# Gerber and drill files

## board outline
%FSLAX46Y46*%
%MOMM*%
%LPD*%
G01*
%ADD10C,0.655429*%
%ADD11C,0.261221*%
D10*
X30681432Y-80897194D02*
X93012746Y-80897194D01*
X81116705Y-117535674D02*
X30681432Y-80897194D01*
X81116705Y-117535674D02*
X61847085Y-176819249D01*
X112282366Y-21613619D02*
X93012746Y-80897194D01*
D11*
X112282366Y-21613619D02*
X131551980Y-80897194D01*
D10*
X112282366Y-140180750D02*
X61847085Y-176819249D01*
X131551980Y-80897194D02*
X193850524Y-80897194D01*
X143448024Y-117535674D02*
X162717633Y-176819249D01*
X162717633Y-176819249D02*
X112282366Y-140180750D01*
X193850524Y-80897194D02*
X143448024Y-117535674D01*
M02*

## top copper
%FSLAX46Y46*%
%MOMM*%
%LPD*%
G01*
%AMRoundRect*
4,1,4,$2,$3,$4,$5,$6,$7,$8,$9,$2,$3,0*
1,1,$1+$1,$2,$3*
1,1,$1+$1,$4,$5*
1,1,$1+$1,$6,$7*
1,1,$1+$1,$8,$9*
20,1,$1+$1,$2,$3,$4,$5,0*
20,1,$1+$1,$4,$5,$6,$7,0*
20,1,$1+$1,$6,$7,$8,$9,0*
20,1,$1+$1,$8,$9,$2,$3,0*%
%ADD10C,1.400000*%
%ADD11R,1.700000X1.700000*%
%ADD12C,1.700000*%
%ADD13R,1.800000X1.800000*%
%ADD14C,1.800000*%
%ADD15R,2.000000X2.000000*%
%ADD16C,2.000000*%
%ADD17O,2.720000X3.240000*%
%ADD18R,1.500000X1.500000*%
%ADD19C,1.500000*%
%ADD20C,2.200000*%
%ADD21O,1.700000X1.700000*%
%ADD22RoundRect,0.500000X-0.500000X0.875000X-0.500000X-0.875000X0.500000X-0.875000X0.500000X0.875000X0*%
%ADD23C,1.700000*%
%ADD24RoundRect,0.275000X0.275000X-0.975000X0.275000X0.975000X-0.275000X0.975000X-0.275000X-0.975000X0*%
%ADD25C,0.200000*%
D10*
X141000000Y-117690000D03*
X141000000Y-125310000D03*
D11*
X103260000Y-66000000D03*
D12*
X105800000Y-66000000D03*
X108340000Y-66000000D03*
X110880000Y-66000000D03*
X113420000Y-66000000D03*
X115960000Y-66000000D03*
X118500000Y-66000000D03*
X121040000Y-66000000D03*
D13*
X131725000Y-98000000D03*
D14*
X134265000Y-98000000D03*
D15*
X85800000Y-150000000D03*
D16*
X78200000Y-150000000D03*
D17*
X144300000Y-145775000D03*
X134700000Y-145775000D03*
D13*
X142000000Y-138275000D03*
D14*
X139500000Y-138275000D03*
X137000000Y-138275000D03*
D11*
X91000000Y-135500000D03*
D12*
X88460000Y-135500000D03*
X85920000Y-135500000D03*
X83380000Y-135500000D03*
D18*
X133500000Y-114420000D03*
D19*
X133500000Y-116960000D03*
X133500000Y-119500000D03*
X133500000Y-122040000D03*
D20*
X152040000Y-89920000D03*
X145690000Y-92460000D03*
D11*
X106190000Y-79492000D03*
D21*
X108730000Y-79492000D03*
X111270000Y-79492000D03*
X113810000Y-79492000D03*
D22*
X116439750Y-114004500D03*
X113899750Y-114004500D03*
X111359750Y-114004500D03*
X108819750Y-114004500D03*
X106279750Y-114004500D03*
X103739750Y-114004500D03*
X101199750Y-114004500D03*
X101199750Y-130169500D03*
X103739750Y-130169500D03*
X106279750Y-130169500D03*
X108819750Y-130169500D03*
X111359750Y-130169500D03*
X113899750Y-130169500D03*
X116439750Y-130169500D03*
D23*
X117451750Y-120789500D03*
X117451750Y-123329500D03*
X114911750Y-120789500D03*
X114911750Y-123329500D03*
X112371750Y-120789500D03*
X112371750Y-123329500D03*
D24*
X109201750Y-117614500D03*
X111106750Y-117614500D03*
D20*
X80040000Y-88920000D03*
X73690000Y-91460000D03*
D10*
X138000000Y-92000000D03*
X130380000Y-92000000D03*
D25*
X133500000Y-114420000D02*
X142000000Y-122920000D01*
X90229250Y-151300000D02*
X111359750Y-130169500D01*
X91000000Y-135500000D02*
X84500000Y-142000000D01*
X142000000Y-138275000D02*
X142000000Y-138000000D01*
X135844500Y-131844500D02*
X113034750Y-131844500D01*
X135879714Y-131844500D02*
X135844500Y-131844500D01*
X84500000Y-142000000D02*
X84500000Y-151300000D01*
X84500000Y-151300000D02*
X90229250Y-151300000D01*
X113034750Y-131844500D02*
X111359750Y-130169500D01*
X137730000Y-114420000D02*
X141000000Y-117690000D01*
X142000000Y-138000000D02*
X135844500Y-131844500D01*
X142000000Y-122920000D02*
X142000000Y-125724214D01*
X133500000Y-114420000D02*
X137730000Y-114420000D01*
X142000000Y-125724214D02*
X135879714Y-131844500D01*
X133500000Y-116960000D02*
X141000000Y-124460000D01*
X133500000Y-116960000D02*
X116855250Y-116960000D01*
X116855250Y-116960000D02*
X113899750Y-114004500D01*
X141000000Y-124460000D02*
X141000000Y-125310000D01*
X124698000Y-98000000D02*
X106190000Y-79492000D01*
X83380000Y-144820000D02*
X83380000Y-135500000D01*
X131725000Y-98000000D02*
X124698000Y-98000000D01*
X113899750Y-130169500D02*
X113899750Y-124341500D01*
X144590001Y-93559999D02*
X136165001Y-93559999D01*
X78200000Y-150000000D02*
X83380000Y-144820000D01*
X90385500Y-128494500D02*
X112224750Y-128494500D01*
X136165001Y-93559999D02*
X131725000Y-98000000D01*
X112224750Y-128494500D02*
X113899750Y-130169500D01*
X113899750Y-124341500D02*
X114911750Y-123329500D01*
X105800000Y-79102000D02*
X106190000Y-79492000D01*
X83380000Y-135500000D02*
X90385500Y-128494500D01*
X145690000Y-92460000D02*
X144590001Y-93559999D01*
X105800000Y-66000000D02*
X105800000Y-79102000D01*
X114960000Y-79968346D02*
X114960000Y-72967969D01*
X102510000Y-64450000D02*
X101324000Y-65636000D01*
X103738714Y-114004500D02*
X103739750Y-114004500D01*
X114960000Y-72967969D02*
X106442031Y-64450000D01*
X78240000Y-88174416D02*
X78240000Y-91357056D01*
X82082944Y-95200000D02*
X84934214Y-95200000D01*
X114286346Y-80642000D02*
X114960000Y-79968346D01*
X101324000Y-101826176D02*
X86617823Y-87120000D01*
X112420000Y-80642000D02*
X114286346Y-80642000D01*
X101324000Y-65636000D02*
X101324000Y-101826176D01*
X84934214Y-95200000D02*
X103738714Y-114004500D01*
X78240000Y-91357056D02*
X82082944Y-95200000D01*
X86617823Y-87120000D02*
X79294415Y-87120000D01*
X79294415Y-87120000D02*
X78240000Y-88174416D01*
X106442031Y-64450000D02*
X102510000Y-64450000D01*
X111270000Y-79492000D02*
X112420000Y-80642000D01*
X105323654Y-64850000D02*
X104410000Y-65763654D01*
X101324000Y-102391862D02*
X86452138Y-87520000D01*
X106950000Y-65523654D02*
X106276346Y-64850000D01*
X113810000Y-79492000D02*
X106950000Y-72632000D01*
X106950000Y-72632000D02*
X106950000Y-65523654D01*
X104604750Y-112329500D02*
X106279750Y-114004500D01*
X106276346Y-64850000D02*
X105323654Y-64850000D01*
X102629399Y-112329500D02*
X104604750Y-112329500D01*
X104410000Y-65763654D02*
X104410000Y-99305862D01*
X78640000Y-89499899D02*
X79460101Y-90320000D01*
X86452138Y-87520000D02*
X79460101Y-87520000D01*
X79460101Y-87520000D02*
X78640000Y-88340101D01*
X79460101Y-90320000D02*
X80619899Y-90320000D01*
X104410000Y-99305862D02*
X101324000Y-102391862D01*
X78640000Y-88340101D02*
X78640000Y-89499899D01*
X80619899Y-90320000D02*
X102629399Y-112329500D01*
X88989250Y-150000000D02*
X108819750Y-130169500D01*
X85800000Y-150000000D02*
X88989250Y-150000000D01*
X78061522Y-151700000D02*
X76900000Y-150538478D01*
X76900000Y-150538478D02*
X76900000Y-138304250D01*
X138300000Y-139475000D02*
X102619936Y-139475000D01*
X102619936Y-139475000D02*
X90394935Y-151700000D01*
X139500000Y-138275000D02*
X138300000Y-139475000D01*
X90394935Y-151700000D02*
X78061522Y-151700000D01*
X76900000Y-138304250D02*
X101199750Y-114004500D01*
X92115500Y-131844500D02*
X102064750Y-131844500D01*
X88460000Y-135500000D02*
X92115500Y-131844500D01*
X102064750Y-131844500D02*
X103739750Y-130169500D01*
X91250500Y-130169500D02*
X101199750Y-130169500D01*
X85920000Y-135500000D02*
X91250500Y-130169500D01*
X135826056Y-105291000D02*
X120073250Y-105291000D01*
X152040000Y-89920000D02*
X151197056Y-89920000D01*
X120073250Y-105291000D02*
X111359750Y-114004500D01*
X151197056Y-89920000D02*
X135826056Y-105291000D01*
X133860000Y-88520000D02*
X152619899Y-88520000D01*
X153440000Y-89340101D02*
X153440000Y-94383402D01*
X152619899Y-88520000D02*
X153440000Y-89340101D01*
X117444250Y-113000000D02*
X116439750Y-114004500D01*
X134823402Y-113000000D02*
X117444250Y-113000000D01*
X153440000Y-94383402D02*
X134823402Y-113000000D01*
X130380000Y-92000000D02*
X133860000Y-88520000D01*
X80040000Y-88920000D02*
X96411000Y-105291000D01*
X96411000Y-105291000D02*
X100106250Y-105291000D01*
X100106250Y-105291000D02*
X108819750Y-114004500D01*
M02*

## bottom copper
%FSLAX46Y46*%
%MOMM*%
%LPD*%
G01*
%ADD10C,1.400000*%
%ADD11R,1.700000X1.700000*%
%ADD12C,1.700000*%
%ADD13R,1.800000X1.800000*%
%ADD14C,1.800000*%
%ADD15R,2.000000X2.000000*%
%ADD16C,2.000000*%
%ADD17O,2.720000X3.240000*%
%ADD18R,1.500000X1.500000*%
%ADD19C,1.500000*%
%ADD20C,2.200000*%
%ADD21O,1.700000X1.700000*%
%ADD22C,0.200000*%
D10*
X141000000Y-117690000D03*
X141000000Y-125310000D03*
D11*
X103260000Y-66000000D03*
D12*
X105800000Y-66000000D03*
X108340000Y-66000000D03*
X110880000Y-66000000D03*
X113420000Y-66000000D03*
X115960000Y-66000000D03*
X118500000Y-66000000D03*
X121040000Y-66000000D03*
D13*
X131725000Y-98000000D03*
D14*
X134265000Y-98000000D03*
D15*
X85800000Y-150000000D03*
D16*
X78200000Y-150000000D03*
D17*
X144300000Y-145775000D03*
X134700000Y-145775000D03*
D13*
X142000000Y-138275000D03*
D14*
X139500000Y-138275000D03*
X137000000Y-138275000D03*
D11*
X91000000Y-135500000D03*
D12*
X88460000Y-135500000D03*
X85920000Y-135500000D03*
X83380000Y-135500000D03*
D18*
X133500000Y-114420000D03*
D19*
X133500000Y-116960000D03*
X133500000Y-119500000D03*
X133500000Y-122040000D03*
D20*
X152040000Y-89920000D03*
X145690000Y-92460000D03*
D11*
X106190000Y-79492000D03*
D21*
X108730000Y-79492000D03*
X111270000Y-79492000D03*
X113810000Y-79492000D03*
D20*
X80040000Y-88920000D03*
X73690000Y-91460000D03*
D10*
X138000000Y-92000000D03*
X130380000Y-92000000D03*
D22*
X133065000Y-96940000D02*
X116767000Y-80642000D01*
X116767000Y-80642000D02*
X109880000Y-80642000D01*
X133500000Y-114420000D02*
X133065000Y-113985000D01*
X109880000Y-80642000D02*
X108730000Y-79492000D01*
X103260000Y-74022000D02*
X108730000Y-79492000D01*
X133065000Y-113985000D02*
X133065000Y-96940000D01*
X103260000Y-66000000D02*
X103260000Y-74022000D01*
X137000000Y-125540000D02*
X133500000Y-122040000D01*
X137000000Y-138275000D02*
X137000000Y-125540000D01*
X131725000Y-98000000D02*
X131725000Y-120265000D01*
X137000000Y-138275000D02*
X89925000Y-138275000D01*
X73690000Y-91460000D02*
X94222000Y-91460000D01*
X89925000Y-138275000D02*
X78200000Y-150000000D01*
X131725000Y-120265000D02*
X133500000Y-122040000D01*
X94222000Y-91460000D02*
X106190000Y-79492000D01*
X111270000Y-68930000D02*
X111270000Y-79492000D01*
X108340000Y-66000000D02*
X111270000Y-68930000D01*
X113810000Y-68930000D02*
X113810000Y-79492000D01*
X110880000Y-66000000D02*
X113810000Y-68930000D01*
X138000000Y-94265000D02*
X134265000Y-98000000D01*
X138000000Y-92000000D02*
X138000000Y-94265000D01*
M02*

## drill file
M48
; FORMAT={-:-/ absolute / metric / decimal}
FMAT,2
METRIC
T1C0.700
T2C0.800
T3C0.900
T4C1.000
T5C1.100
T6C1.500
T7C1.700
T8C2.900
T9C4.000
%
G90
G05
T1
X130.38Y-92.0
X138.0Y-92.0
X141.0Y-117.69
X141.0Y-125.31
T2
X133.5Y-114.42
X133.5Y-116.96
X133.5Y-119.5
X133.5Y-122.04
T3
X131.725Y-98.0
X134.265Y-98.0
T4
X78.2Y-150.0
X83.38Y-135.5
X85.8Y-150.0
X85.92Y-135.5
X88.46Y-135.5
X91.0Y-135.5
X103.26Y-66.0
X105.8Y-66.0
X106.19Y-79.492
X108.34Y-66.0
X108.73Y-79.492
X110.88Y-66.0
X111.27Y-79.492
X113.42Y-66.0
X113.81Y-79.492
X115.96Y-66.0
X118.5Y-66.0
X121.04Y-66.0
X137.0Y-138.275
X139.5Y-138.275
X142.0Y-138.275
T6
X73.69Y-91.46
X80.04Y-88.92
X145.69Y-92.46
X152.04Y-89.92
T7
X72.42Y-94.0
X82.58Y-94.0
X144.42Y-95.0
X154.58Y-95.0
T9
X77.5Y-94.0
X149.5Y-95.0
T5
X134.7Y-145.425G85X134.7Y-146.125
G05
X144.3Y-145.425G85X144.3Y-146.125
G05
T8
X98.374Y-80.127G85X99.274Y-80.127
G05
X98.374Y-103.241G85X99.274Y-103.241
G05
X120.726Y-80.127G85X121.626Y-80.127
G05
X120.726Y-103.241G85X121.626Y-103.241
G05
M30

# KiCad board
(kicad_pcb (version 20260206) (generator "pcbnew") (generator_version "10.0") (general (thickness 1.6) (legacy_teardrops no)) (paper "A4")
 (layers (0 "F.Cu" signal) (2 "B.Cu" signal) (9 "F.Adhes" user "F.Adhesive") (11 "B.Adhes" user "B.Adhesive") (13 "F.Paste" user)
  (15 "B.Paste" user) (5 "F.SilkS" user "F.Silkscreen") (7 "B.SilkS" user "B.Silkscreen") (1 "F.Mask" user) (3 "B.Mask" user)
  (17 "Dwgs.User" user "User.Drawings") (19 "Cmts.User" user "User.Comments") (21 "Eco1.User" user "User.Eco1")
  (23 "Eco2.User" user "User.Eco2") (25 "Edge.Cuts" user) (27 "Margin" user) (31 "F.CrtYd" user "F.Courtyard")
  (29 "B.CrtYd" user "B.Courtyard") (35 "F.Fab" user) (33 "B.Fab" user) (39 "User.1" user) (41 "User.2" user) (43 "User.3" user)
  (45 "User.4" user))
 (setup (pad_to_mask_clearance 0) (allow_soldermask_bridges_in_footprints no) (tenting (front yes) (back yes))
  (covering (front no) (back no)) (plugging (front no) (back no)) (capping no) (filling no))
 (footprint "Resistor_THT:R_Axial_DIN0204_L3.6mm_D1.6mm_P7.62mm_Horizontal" (layer "F.Cu") (at 141 117.69 -90)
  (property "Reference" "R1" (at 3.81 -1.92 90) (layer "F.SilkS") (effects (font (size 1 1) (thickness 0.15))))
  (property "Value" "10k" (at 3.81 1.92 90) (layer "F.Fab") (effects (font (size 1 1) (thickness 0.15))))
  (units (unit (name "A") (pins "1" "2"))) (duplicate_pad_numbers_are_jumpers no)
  (pad "1" thru_hole circle (at 0 0 270) (size 1.4 1.4) (drill 0.7) (layers "*.Cu" "*.Mask") (remove_unused_layers no) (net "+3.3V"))
  (pad "2" thru_hole circle (at 7.62 0 270) (size 1.4 1.4) (drill 0.7) (layers "*.Cu" "*.Mask") (remove_unused_layers no)
   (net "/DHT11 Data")))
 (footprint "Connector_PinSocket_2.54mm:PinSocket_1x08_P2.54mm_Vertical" (layer "F.Cu") (at 103.26 66 90)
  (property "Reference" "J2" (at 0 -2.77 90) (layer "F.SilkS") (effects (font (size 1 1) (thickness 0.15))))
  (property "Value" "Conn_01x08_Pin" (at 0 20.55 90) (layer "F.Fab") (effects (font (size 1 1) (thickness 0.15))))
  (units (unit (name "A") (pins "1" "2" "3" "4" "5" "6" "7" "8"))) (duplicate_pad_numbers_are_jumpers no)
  (pad "1" thru_hole rect (at 0 0 90) (size 1.7 1.7) (drill 1) (layers "*.Cu" "*.Mask") (remove_unused_layers no) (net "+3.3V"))
  (pad "2" thru_hole circle (at 0 2.54 90) (size 1.7 1.7) (drill 1) (layers "*.Cu" "*.Mask") (remove_unused_layers no) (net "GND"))
  (pad "3" thru_hole circle (at 0 5.08 90) (size 1.7 1.7) (drill 1) (layers "*.Cu" "*.Mask") (remove_unused_layers no) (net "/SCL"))
  (pad "4" thru_hole circle (at 0 7.62 90) (size 1.7 1.7) (drill 1) (layers "*.Cu" "*.Mask") (remove_unused_layers no) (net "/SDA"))
  (pad "5" thru_hole circle (at 0 10.16 90) (size 1.7 1.7) (drill 1) (layers "*.Cu" "*.Mask") (remove_unused_layers no)
   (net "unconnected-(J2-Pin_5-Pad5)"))
  (pad "6" thru_hole circle (at 0 12.7 90) (size 1.7 1.7) (drill 1) (layers "*.Cu" "*.Mask") (remove_unused_layers no)
   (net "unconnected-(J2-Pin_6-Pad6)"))
  (pad "7" thru_hole circle (at 0 15.24 90) (size 1.7 1.7) (drill 1) (layers "*.Cu" "*.Mask") (remove_unused_layers no)
   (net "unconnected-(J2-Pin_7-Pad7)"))
  (pad "8" thru_hole circle (at 0 17.78 90) (size 1.7 1.7) (drill 1) (layers "*.Cu" "*.Mask") (remove_unused_layers no)
   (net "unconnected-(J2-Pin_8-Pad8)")))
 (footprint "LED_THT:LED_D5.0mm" (layer "F.Cu") (at 131.725 98)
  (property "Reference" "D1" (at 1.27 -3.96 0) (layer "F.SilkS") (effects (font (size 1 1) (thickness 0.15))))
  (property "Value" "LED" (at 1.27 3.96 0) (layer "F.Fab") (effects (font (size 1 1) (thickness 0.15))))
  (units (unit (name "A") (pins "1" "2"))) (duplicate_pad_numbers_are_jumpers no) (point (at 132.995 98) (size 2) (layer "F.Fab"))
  (pad "1" thru_hole rect (at 0 0) (size 1.8 1.8) (drill 0.9) (layers "*.Cu" "*.Mask") (remove_unused_layers no) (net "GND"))
  (pad "2" thru_hole circle (at 2.54 0) (size 1.8 1.8) (drill 0.9) (layers "*.Cu" "*.Mask") (remove_unused_layers no) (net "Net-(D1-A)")))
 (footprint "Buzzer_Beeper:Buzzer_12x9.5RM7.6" (layer "F.Cu") (at 85.8 150 180)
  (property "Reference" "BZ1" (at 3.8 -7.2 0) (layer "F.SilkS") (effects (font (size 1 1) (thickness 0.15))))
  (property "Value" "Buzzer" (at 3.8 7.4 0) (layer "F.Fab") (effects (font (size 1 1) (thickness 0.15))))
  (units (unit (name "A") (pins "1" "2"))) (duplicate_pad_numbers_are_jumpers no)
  (pad "1" thru_hole rect (at 0 0 180) (size 2 2) (drill 1) (layers "*.Cu" "*.Mask") (remove_unused_layers no) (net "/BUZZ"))
  (pad "2" thru_hole circle (at 7.6 0 180) (size 2 2) (drill 1) (layers "*.Cu" "*.Mask") (remove_unused_layers no) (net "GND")))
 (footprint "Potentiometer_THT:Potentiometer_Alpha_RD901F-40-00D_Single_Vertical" (layer "F.Cu") (at 142 138.275 -90)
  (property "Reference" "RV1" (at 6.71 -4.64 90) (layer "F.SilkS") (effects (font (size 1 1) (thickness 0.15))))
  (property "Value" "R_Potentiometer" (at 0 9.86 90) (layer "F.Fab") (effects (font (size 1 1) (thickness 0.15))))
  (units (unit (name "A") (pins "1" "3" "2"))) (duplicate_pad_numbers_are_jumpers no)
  (pad "" thru_hole oval (at 7.5 -2.3) (size 2.72 3.24) (drill oval 1.1 1.8) (layers "*.Cu" "*.Mask") (remove_unused_layers no))
  (pad "" thru_hole oval (at 7.5 7.3) (size 2.72 3.24) (drill oval 1.1 1.8) (layers "*.Cu" "*.Mask") (remove_unused_layers no))
  (pad "1" thru_hole rect (at 0 0) (size 1.8 1.8) (drill 1) (layers "*.Cu" "*.Mask") (remove_unused_layers no) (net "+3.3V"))
  (pad "2" thru_hole circle (at 0 2.5) (size 1.8 1.8) (drill 1) (layers "*.Cu" "*.Mask") (remove_unused_layers no) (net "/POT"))
  (pad "3" thru_hole circle (at 0 5) (size 1.8 1.8) (drill 1) (layers "*.Cu" "*.Mask") (remove_unused_layers no) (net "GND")))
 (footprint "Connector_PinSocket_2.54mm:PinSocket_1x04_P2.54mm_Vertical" (layer "F.Cu") (at 91 135.5 -90)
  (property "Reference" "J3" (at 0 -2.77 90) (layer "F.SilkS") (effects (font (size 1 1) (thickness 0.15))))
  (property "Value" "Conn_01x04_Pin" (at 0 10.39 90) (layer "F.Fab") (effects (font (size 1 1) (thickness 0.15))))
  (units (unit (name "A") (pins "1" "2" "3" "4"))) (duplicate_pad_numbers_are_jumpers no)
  (pad "1" thru_hole rect (at 0 0 270) (size 1.7 1.7) (drill 1) (layers "*.Cu" "*.Mask") (remove_unused_layers no) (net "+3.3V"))
  (pad "2" thru_hole circle (at 0 2.54 270) (size 1.7 1.7) (drill 1) (layers "*.Cu" "*.Mask") (remove_unused_layers no) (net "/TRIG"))
  (pad "3" thru_hole circle (at 0 5.08 270) (size 1.7 1.7) (drill 1) (layers "*.Cu" "*.Mask") (remove_unused_layers no) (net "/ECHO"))
  (pad "4" thru_hole circle (at 0 7.62 270) (size 1.7 1.7) (drill 1) (layers "*.Cu" "*.Mask") (remove_unused_layers no) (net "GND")))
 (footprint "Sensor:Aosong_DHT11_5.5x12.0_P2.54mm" (layer "F.Cu") (at 133.5 114.42)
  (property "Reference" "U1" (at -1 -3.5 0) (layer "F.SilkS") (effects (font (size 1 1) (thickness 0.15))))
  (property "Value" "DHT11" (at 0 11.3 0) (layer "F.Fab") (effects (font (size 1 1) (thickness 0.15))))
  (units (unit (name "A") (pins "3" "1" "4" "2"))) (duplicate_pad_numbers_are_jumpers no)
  (pad "1" thru_hole rect (at 0 0) (size 1.5 1.5) (drill 0.8) (layers "*.Cu" "*.Mask") (remove_unused_layers no) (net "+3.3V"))
  (pad "2" thru_hole circle (at 0 2.54) (size 1.5 1.5) (drill 0.8) (layers "*.Cu" "*.Mask") (remove_unused_layers no) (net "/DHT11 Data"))
  (pad "3" thru_hole circle (at 0 5.08) (size 1.5 1.5) (drill 0.8) (layers "*.Cu" "*.Mask") (remove_unused_layers no)
   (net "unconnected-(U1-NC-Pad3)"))
  (pad "4" thru_hole circle (at 0 7.62) (size 1.5 1.5) (drill 0.8) (layers "*.Cu" "*.Mask") (remove_unused_layers no) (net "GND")))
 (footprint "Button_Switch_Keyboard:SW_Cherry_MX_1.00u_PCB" (layer "F.Cu") (at 152.04 89.92)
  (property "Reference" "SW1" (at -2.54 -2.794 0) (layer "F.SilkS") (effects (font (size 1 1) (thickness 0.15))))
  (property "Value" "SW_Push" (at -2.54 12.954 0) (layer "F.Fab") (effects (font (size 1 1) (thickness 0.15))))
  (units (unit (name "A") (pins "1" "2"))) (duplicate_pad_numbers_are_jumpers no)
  (pad "" np_thru_hole circle (at -7.62 5.08) (size 1.7 1.7) (drill 1.7) (layers "*.Cu" "*.Mask"))
  (pad "" np_thru_hole circle (at -2.54 5.08) (size 4 4) (drill 4) (layers "*.Cu" "*.Mask"))
  (pad "" np_thru_hole circle (at 2.54 5.08) (size 1.7 1.7) (drill 1.7) (layers "*.Cu" "*.Mask"))
  (pad "1" thru_hole circle (at 0 0) (size 2.2 2.2) (drill 1.5) (layers "*.Cu" "*.Mask") (remove_unused_layers no) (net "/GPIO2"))
  (pad "2" thru_hole circle (at -6.35 2.54) (size 2.2 2.2) (drill 1.5) (layers "*.Cu" "*.Mask") (remove_unused_layers no) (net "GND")))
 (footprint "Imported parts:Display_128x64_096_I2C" (layer "F.Cu") (at 110 79.492)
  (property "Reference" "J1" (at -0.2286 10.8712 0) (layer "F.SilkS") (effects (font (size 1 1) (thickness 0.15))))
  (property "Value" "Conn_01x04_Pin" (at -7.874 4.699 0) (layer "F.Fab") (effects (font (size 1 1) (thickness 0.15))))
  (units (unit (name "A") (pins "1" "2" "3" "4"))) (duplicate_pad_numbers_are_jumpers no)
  (pad "" np_thru_hole oval (at -11.176 0.635) (size 3.8 2.9) (drill oval 3.8 2.9) (layers "*.Cu" "*.Mask"))
  (pad "" np_thru_hole oval (at -11.176 23.749) (size 3.8 2.9) (drill oval 3.8 2.9) (layers "*.Cu" "*.Mask"))
  (pad "" np_thru_hole oval (at 11.176 0.635) (size 3.8 2.9) (drill oval 3.8 2.9) (layers "*.Cu" "*.Mask"))
  (pad "" np_thru_hole oval (at 11.176 23.749) (size 3.8 2.9) (drill oval 3.8 2.9) (layers "*.Cu" "*.Mask"))
  (pad "1" thru_hole rect (at -3.81 0 90) (size 1.7 1.7) (drill 1) (layers "*.Cu" "*.Mask") (remove_unused_layers no) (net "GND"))
  (pad "2" thru_hole oval (at -1.27 0 90) (size 1.7 1.7) (drill 1) (layers "*.Cu" "*.Mask") (remove_unused_layers no) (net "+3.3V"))
  (pad "3" thru_hole oval (at 1.27 0 90) (size 1.7 1.7) (drill 1) (layers "*.Cu" "*.Mask") (remove_unused_layers no) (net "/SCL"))
  (pad "4" thru_hole oval (at 3.81 0 90) (size 1.7 1.7) (drill 1) (layers "*.Cu" "*.Mask") (remove_unused_layers no) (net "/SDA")))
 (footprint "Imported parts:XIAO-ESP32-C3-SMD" (layer "F.Cu") (at 98.31975 113.1695 -90)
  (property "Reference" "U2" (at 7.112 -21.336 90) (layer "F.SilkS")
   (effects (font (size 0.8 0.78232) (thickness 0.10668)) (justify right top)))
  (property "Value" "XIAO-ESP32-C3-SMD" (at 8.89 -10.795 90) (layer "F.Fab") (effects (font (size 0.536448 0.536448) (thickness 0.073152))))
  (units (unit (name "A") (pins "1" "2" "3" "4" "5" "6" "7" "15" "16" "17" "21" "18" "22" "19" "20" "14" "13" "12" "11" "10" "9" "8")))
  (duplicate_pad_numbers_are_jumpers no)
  (pad "1" smd roundrect (at 0.835 -18.12 270) (size 2.75 2) (layers "F.Cu" "F.Mask" "F.Paste") (roundrect_rratio 0.25) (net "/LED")
   (solder_mask_margin 0.0508) (thermal_bridge_angle 45))
  (pad "2" smd roundrect (at 0.835 -15.58 270) (size 2.75 2) (layers "F.Cu" "F.Mask" "F.Paste") (roundrect_rratio 0.25) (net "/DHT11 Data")
   (solder_mask_margin 0.0508) (thermal_bridge_angle 45))
  (pad "3" smd roundrect (at 0.835 -13.04 270) (size 2.75 2) (layers "F.Cu" "F.Mask" "F.Paste") (roundrect_rratio 0.25) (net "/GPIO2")
   (solder_mask_margin 0.0508) (thermal_bridge_angle 45))
  (pad "4" smd roundrect (at 0.835 -10.5 270) (size 2.75 2) (layers "F.Cu" "F.Mask" "F.Paste") (roundrect_rratio 0.25) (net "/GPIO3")
   (solder_mask_margin 0.0508) (thermal_bridge_angle 45))
  (pad "5" smd roundrect (at 0.835 -7.96 270) (size 2.75 2) (layers "F.Cu" "F.Mask" "F.Paste") (roundrect_rratio 0.25) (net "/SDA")
   (solder_mask_margin 0.0508) (thermal_bridge_angle 45))
  (pad "6" smd roundrect (at 0.835 -5.42 270) (size 2.75 2) (layers "F.Cu" "F.Mask" "F.Paste") (roundrect_rratio 0.25) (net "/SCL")
   (solder_mask_margin 0.0508) (thermal_bridge_angle 45))
  (pad "7" smd roundrect (at 0.835 -2.88 270) (size 2.75 2) (layers "F.Cu" "F.Mask" "F.Paste") (roundrect_rratio 0.25) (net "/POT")
   (solder_mask_margin 0.0508) (thermal_bridge_angle 45))
  (pad "8" smd roundrect (at 17 -2.88 270) (size 2.75 2) (layers "F.Cu" "F.Mask" "F.Paste") (roundrect_rratio 0.25) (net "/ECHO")
   (solder_mask_margin 0.0508) (thermal_bridge_angle 45))
  (pad "9" smd roundrect (at 17 -5.42 270) (size 2.75 2) (layers "F.Cu" "F.Mask" "F.Paste") (roundrect_rratio 0.25) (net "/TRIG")
   (solder_mask_margin 0.0508) (thermal_bridge_angle 45))
  (pad "10" smd roundrect (at 17 -7.96 270) (size 2.75 2) (layers "F.Cu" "F.Mask" "F.Paste") (roundrect_rratio 0.25)
   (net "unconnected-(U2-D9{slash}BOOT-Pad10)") (solder_mask_margin 0.0508) (thermal_bridge_angle 45))
  (pad "11" smd roundrect (at 17 -10.5 270) (size 2.75 2) (layers "F.Cu" "F.Mask" "F.Paste") (roundrect_rratio 0.25) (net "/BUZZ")
   (solder_mask_margin 0.0508) (thermal_bridge_angle 45))
  (pad "12" smd roundrect (at 17 -13.04 270) (size 2.75 2) (layers "F.Cu" "F.Mask" "F.Paste") (roundrect_rratio 0.25) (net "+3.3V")
   (solder_mask_margin 0.0508) (thermal_bridge_angle 45))
  (pad "13" smd roundrect (at 17 -15.58 270) (size 2.75 2) (layers "F.Cu" "F.Mask" "F.Paste") (roundrect_rratio 0.25) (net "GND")
   (solder_mask_margin 0.0508) (thermal_bridge_angle 45))
  (pad "14" smd roundrect (at 17 -18.12 270) (size 2.75 2) (layers "F.Cu" "F.Mask" "F.Paste") (roundrect_rratio 0.25) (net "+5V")
   (solder_mask_margin 0.0508) (thermal_bridge_angle 45))
  (pad "15" smd circle (at 7.62 -19.132 270) (size 1.7 1.7) (layers "F.Cu" "F.Mask" "F.Paste") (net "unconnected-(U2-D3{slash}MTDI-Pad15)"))
  (pad "16" smd circle (at 10.16 -19.132 270) (size 1.7 1.7) (layers "F.Cu" "F.Mask" "F.Paste") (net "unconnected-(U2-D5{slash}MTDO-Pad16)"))
  (pad "17" smd circle (at 7.62 -16.592 270) (size 1.7 1.7) (layers "F.Cu" "F.Mask" "F.Paste") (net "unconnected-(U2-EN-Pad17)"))
  (pad "18" smd circle (at 10.16 -16.592 270) (size 1.7 1.7) (layers "F.Cu" "F.Mask" "F.Paste") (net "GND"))
  (pad "19" smd circle (at 7.62 -14.052 270) (size 1.7 1.7) (layers "F.Cu" "F.Mask" "F.Paste") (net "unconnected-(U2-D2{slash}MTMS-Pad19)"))
  (pad "20" smd circle (at 10.16 -14.052 270) (size 1.7 1.7) (layers "F.Cu" "F.Mask" "F.Paste") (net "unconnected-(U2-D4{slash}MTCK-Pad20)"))
  (pad "21" smd roundrect (at 4.445 -10.882 90) (size 2.5 1.1) (layers "F.Cu" "F.Mask" "F.Paste") (roundrect_rratio 0.25)
   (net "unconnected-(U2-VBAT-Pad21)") (thermal_bridge_angle 45))
  (pad "22" smd roundrect (at 4.445 -12.787 90) (size 2.5 1.1) (layers "F.Cu" "F.Mask" "F.Paste") (roundrect_rratio 0.25)
   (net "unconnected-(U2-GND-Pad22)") (thermal_bridge_angle 45)))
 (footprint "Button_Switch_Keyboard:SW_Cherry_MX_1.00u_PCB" (layer "F.Cu") (at 80.04 88.92)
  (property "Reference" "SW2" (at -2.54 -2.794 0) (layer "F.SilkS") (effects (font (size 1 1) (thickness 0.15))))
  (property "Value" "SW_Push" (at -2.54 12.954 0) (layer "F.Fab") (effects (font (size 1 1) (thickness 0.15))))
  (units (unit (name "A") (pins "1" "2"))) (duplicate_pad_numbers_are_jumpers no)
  (pad "" np_thru_hole circle (at -7.62 5.08) (size 1.7 1.7) (drill 1.7) (layers "*.Cu" "*.Mask"))
  (pad "" np_thru_hole circle (at -2.54 5.08) (size 4 4) (drill 4) (layers "*.Cu" "*.Mask"))
  (pad "" np_thru_hole circle (at 2.54 5.08) (size 1.7 1.7) (drill 1.7) (layers "*.Cu" "*.Mask"))
  (pad "1" thru_hole circle (at 0 0) (size 2.2 2.2) (drill 1.5) (layers "*.Cu" "*.Mask") (remove_unused_layers no) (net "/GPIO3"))
  (pad "2" thru_hole circle (at -6.35 2.54) (size 2.2 2.2) (drill 1.5) (layers "*.Cu" "*.Mask") (remove_unused_layers no) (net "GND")))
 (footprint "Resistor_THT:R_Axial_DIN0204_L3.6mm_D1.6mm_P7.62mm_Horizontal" (layer "F.Cu") (at 138 92 180)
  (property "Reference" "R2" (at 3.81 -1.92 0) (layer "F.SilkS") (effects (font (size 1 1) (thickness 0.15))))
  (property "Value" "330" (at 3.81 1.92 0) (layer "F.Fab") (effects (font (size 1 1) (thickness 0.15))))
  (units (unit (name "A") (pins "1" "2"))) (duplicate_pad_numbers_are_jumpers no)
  (pad "1" thru_hole circle (at 0 0 180) (size 1.4 1.4) (drill 0.7) (layers "*.Cu" "*.Mask") (remove_unused_layers no) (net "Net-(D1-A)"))
  (pad "2" thru_hole circle (at 7.62 0 180) (size 1.4 1.4) (drill 0.7) (layers "*.Cu" "*.Mask") (remove_unused_layers no) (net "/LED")))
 (gr_line (start 30.681432 80.897194) (end 93.012746 80.897194) (stroke (width 0.655429) (type default)) (layer "Edge.Cuts"))
 (gr_line (start 81.116705 117.535674) (end 30.681432 80.897194) (stroke (width 0.655429) (type default)) (layer "Edge.Cuts"))
 (gr_line (start 81.116705 117.535674) (end 61.847085 176.819249) (stroke (width 0.655429) (type default)) (layer "Edge.Cuts"))
 (gr_line (start 112.282366 21.613619) (end 93.012746 80.897194) (stroke (width 0.655429) (type default)) (layer "Edge.Cuts"))
 (gr_line (start 112.282366 21.613619) (end 131.55198 80.897194) (stroke (width 0.261221) (type default)) (layer "Edge.Cuts"))
 (gr_line (start 112.282366 140.18075) (end 61.847085 176.819249) (stroke (width 0.655429) (type default)) (layer "Edge.Cuts"))
 (gr_line (start 131.55198 80.897194) (end 193.850524 80.897194) (stroke (width 0.655429) (type default)) (layer "Edge.Cuts"))
 (gr_line (start 143.448024 117.535674) (end 162.717633 176.819249) (stroke (width 0.655429) (type default)) (layer "Edge.Cuts"))
 (gr_line (start 162.717633 176.819249) (end 112.282366 140.18075) (stroke (width 0.655429) (type default)) (layer "Edge.Cuts"))
 (gr_line (start 193.850524 80.897194) (end 143.448024 117.535674) (stroke (width 0.655429) (type default)) (layer "Edge.Cuts"))
 (segment (start 133.5 114.42) (end 142 122.92) (width 0.2) (layer "F.Cu") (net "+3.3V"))
 (segment (start 90.22925 151.3) (end 111.35975 130.1695) (width 0.2) (layer "F.Cu") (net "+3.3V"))
 (segment (start 91 135.5) (end 84.5 142) (width 0.2) (layer "F.Cu") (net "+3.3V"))
 (segment (start 142 138.275) (end 142 138) (width 0.2) (layer "F.Cu") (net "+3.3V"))
 (segment (start 135.8445 131.8445) (end 113.03475 131.8445) (width 0.2) (layer "F.Cu") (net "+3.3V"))
 (segment (start 135.879714 131.8445) (end 135.8445 131.8445) (width 0.2) (layer "F.Cu") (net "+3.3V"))
 (segment (start 84.5 142) (end 84.5 151.3) (width 0.2) (layer "F.Cu") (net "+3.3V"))
 (segment (start 84.5 151.3) (end 90.22925 151.3) (width 0.2) (layer "F.Cu") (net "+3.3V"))
 (segment (start 113.03475 131.8445) (end 111.35975 130.1695) (width 0.2) (layer "F.Cu") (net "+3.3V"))
 (segment (start 137.73 114.42) (end 141 117.69) (width 0.2) (layer "F.Cu") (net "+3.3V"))
 (segment (start 142 138) (end 135.8445 131.8445) (width 0.2) (layer "F.Cu") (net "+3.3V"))
 (segment (start 142 122.92) (end 142 125.724214) (width 0.2) (layer "F.Cu") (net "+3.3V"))
 (segment (start 133.5 114.42) (end 137.73 114.42) (width 0.2) (layer "F.Cu") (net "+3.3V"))
 (segment (start 142 125.724214) (end 135.879714 131.8445) (width 0.2) (layer "F.Cu") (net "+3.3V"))
 (segment (start 133.065 96.94) (end 116.767 80.642) (width 0.2) (layer "B.Cu") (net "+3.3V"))
 (segment (start 116.767 80.642) (end 109.88 80.642) (width 0.2) (layer "B.Cu") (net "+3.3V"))
 (segment (start 133.5 114.42) (end 133.065 113.985) (width 0.2) (layer "B.Cu") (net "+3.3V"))
 (segment (start 109.88 80.642) (end 108.73 79.492) (width 0.2) (layer "B.Cu") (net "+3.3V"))
 (segment (start 103.26 74.022) (end 108.73 79.492) (width 0.2) (layer "B.Cu") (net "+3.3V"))
 (segment (start 133.065 113.985) (end 133.065 96.94) (width 0.2) (layer "B.Cu") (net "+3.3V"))
 (segment (start 103.26 66) (end 103.26 74.022) (width 0.2) (layer "B.Cu") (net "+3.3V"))
 (segment (start 133.5 116.96) (end 141 124.46) (width 0.2) (layer "F.Cu") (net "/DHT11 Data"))
 (segment (start 133.5 116.96) (end 116.85525 116.96) (width 0.2) (layer "F.Cu") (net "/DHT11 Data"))
 (segment (start 116.85525 116.96) (end 113.89975 114.0045) (width 0.2) (layer "F.Cu") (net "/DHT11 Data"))
 (segment (start 141 124.46) (end 141 125.31) (width 0.2) (layer "F.Cu") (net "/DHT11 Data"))
 (segment (start 124.698 98) (end 106.19 79.492) (width 0.2) (layer "F.Cu") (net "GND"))
 (segment (start 83.38 144.82) (end 83.38 135.5) (width 0.2) (layer "F.Cu") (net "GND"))
 (segment (start 131.725 98) (end 124.698 98) (width 0.2) (layer "F.Cu") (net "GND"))
 (segment (start 113.89975 130.1695) (end 113.89975 124.3415) (width 0.2) (layer "F.Cu") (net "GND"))
 (segment (start 144.590001 93.559999) (end 136.165001 93.559999) (width 0.2) (layer "F.Cu") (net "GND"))
 (segment (start 78.2 150) (end 83.38 144.82) (width 0.2) (layer "F.Cu") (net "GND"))
 (segment (start 90.3855 128.4945) (end 112.22475 128.4945) (width 0.2) (layer "F.Cu") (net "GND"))
 (segment (start 136.165001 93.559999) (end 131.725 98) (width 0.2) (layer "F.Cu") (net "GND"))
 (segment (start 112.22475 128.4945) (end 113.89975 130.1695) (width 0.2) (layer "F.Cu") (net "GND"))
 (segment (start 113.89975 124.3415) (end 114.91175 123.3295) (width 0.2) (layer "F.Cu") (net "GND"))
 (segment (start 105.8 79.102) (end 106.19 79.492) (width 0.2) (layer "F.Cu") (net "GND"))
 (segment (start 83.38 135.5) (end 90.3855 128.4945) (width 0.2) (layer "F.Cu") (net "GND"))
 (segment (start 145.69 92.46) (end 144.590001 93.559999) (width 0.2) (layer "F.Cu") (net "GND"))
 (segment (start 105.8 66) (end 105.8 79.102) (width 0.2) (layer "F.Cu") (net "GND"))
 (segment (start 137 125.54) (end 133.5 122.04) (width 0.2) (layer "B.Cu") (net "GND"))
 (segment (start 137 138.275) (end 137 125.54) (width 0.2) (layer "B.Cu") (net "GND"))
 (segment (start 131.725 98) (end 131.725 120.265) (width 0.2) (layer "B.Cu") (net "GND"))
 (segment (start 137 138.275) (end 89.925 138.275) (width 0.2) (layer "B.Cu") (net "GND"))
 (segment (start 73.69 91.46) (end 94.222 91.46) (width 0.2) (layer "B.Cu") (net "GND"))
 (segment (start 89.925 138.275) (end 78.2 150) (width 0.2) (layer "B.Cu") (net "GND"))
 (segment (start 131.725 120.265) (end 133.5 122.04) (width 0.2) (layer "B.Cu") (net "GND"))
 (segment (start 94.222 91.46) (end 106.19 79.492) (width 0.2) (layer "B.Cu") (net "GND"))
 (segment (start 114.96 79.968346) (end 114.96 72.967969) (width 0.2) (layer "F.Cu") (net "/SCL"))
 (segment (start 102.51 64.45) (end 101.324 65.636) (width 0.2) (layer "F.Cu") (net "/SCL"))
 (segment (start 103.738714 114.0045) (end 103.73975 114.0045) (width 0.2) (layer "F.Cu") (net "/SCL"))
 (segment (start 114.96 72.967969) (end 106.442031 64.45) (width 0.2) (layer "F.Cu") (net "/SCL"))
 (segment (start 78.24 88.174416) (end 78.24 91.357056) (width 0.2) (layer "F.Cu") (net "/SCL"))
 (segment (start 82.082944 95.2) (end 84.934214 95.2) (width 0.2) (layer "F.Cu") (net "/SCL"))
 (segment (start 114.286346 80.642) (end 114.96 79.968346) (width 0.2) (layer "F.Cu") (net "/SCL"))
 (segment (start 101.324 101.826176) (end 86.617823 87.12) (width 0.2) (layer "F.Cu") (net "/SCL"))
 (segment (start 112.42 80.642) (end 114.286346 80.642) (width 0.2) (layer "F.Cu") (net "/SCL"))
 (segment (start 101.324 65.636) (end 101.324 101.826176) (width 0.2) (layer "F.Cu") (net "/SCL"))
 (segment (start 84.934214 95.2) (end 103.738714 114.0045) (width 0.2) (layer "F.Cu") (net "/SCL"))
 (segment (start 78.24 91.357056) (end 82.082944 95.2) (width 0.2) (layer "F.Cu") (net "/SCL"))
 (segment (start 86.617823 87.12) (end 79.294415 87.12) (width 0.2) (layer "F.Cu") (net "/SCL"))
 (segment (start 79.294415 87.12) (end 78.24 88.174416) (width 0.2) (layer "F.Cu") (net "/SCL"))
 (segment (start 106.442031 64.45) (end 102.51 64.45) (width 0.2) (layer "F.Cu") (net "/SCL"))
 (segment (start 111.27 79.492) (end 112.42 80.642) (width 0.2) (layer "F.Cu") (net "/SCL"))
 (segment (start 111.27 68.93) (end 111.27 79.492) (width 0.2) (layer "B.Cu") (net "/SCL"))
 (segment (start 108.34 66) (end 111.27 68.93) (width 0.2) (layer "B.Cu") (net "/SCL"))
 (segment (start 105.323654 64.85) (end 104.41 65.763654) (width 0.2) (layer "F.Cu") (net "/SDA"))
 (segment (start 101.324 102.391862) (end 86.452138 87.52) (width 0.2) (layer "F.Cu") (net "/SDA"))
 (segment (start 106.95 65.523654) (end 106.276346 64.85) (width 0.2) (layer "F.Cu") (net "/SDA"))
 (segment (start 113.81 79.492) (end 106.95 72.632) (width 0.2) (layer "F.Cu") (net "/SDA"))
 (segment (start 106.95 72.632) (end 106.95 65.523654) (width 0.2) (layer "F.Cu") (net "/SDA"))
 (segment (start 104.60475 112.3295) (end 106.27975 114.0045) (width 0.2) (layer "F.Cu") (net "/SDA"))
 (segment (start 106.276346 64.85) (end 105.323654 64.85) (width 0.2) (layer "F.Cu") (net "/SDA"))
 (segment (start 102.629399 112.3295) (end 104.60475 112.3295) (width 0.2) (layer "F.Cu") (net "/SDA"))
 (segment (start 104.41 65.763654) (end 104.41 99.305862) (width 0.2) (layer "F.Cu") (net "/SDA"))
 (segment (start 78.64 89.499899) (end 79.460101 90.32) (width 0.2) (layer "F.Cu") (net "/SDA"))
 (segment (start 86.452138 87.52) (end 79.460101 87.52) (width 0.2) (layer "F.Cu") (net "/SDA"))
 (segment (start 79.460101 87.52) (end 78.64 88.340101) (width 0.2) (layer "F.Cu") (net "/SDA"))
 (segment (start 79.460101 90.32) (end 80.619899 90.32) (width 0.2) (layer "F.Cu") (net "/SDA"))
 (segment (start 104.41 99.305862) (end 101.324 102.391862) (width 0.2) (layer "F.Cu") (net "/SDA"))
 (segment (start 78.64 88.340101) (end 78.64 89.499899) (width 0.2) (layer "F.Cu") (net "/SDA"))
 (segment (start 80.619899 90.32) (end 102.629399 112.3295) (width 0.2) (layer "F.Cu") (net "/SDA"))
 (segment (start 113.81 68.93) (end 113.81 79.492) (width 0.2) (layer "B.Cu") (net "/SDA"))
 (segment (start 110.88 66) (end 113.81 68.93) (width 0.2) (layer "B.Cu") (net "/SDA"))
 (segment (start 138 94.265) (end 134.265 98) (width 0.2) (layer "B.Cu") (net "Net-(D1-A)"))
 (segment (start 138 92) (end 138 94.265) (width 0.2) (layer "B.Cu") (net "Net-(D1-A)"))
 (segment (start 88.98925 150) (end 108.81975 130.1695) (width 0.2) (layer "F.Cu") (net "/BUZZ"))
 (segment (start 85.8 150) (end 88.98925 150) (width 0.2) (layer "F.Cu") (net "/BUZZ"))
 (segment (start 78.061522 151.7) (end 76.9 150.538478) (width 0.2) (layer "F.Cu") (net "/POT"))
 (segment (start 76.9 150.538478) (end 76.9 138.30425) (width 0.2) (layer "F.Cu") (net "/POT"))
 (segment (start 138.3 139.475) (end 102.619936 139.475) (width 0.2) (layer "F.Cu") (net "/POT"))
 (segment (start 102.619936 139.475) (end 90.394935 151.7) (width 0.2) (layer "F.Cu") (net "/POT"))
 (segment (start 139.5 138.275) (end 138.3 139.475) (width 0.2) (layer "F.Cu") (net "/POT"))
 (segment (start 90.394935 151.7) (end 78.061522 151.7) (width 0.2) (layer "F.Cu") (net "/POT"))
 (segment (start 76.9 138.30425) (end 101.19975 114.0045) (width 0.2) (layer "F.Cu") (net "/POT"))
 (segment (start 92.1155 131.8445) (end 102.06475 131.8445) (width 0.2) (layer "F.Cu") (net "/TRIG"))
 (segment (start 88.46 135.5) (end 92.1155 131.8445) (width 0.2) (layer "F.Cu") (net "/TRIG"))
 (segment (start 102.06475 131.8445) (end 103.73975 130.1695) (width 0.2) (layer "F.Cu") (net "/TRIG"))
 (segment (start 91.2505 130.1695) (end 101.19975 130.1695) (width 0.2) (layer "F.Cu") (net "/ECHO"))
 (segment (start 85.92 135.5) (end 91.2505 130.1695) (width 0.2) (layer "F.Cu") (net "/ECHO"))
 (segment (start 135.826056 105.291) (end 120.07325 105.291) (width 0.2) (layer "F.Cu") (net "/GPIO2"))
 (segment (start 152.04 89.92) (end 151.197056 89.92) (width 0.2) (layer "F.Cu") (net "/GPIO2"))
 (segment (start 120.07325 105.291) (end 111.35975 114.0045) (width 0.2) (layer "F.Cu") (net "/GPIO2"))
 (segment (start 151.197056 89.92) (end 135.826056 105.291) (width 0.2) (layer "F.Cu") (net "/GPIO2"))
 (segment (start 133.86 88.52) (end 152.619899 88.52) (width 0.2) (layer "F.Cu") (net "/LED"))
 (segment (start 153.44 89.340101) (end 153.44 94.383402) (width 0.2) (layer "F.Cu") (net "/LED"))
 (segment (start 152.619899 88.52) (end 153.44 89.340101) (width 0.2) (layer "F.Cu") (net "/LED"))
 (segment (start 117.44425 113) (end 116.43975 114.0045) (width 0.2) (layer "F.Cu") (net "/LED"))
 (segment (start 134.823402 113) (end 117.44425 113) (width 0.2) (layer "F.Cu") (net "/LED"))
 (segment (start 153.44 94.383402) (end 134.823402 113) (width 0.2) (layer "F.Cu") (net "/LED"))
 (segment (start 130.38 92) (end 133.86 88.52) (width 0.2) (layer "F.Cu") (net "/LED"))
 (segment (start 80.04 88.92) (end 96.411 105.291) (width 0.2) (layer "F.Cu") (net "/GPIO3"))
 (segment (start 96.411 105.291) (end 100.10625 105.291) (width 0.2) (layer "F.Cu") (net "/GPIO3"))
 (segment (start 100.10625 105.291) (end 108.81975 114.0045) (width 0.2) (layer "F.Cu") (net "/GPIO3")))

